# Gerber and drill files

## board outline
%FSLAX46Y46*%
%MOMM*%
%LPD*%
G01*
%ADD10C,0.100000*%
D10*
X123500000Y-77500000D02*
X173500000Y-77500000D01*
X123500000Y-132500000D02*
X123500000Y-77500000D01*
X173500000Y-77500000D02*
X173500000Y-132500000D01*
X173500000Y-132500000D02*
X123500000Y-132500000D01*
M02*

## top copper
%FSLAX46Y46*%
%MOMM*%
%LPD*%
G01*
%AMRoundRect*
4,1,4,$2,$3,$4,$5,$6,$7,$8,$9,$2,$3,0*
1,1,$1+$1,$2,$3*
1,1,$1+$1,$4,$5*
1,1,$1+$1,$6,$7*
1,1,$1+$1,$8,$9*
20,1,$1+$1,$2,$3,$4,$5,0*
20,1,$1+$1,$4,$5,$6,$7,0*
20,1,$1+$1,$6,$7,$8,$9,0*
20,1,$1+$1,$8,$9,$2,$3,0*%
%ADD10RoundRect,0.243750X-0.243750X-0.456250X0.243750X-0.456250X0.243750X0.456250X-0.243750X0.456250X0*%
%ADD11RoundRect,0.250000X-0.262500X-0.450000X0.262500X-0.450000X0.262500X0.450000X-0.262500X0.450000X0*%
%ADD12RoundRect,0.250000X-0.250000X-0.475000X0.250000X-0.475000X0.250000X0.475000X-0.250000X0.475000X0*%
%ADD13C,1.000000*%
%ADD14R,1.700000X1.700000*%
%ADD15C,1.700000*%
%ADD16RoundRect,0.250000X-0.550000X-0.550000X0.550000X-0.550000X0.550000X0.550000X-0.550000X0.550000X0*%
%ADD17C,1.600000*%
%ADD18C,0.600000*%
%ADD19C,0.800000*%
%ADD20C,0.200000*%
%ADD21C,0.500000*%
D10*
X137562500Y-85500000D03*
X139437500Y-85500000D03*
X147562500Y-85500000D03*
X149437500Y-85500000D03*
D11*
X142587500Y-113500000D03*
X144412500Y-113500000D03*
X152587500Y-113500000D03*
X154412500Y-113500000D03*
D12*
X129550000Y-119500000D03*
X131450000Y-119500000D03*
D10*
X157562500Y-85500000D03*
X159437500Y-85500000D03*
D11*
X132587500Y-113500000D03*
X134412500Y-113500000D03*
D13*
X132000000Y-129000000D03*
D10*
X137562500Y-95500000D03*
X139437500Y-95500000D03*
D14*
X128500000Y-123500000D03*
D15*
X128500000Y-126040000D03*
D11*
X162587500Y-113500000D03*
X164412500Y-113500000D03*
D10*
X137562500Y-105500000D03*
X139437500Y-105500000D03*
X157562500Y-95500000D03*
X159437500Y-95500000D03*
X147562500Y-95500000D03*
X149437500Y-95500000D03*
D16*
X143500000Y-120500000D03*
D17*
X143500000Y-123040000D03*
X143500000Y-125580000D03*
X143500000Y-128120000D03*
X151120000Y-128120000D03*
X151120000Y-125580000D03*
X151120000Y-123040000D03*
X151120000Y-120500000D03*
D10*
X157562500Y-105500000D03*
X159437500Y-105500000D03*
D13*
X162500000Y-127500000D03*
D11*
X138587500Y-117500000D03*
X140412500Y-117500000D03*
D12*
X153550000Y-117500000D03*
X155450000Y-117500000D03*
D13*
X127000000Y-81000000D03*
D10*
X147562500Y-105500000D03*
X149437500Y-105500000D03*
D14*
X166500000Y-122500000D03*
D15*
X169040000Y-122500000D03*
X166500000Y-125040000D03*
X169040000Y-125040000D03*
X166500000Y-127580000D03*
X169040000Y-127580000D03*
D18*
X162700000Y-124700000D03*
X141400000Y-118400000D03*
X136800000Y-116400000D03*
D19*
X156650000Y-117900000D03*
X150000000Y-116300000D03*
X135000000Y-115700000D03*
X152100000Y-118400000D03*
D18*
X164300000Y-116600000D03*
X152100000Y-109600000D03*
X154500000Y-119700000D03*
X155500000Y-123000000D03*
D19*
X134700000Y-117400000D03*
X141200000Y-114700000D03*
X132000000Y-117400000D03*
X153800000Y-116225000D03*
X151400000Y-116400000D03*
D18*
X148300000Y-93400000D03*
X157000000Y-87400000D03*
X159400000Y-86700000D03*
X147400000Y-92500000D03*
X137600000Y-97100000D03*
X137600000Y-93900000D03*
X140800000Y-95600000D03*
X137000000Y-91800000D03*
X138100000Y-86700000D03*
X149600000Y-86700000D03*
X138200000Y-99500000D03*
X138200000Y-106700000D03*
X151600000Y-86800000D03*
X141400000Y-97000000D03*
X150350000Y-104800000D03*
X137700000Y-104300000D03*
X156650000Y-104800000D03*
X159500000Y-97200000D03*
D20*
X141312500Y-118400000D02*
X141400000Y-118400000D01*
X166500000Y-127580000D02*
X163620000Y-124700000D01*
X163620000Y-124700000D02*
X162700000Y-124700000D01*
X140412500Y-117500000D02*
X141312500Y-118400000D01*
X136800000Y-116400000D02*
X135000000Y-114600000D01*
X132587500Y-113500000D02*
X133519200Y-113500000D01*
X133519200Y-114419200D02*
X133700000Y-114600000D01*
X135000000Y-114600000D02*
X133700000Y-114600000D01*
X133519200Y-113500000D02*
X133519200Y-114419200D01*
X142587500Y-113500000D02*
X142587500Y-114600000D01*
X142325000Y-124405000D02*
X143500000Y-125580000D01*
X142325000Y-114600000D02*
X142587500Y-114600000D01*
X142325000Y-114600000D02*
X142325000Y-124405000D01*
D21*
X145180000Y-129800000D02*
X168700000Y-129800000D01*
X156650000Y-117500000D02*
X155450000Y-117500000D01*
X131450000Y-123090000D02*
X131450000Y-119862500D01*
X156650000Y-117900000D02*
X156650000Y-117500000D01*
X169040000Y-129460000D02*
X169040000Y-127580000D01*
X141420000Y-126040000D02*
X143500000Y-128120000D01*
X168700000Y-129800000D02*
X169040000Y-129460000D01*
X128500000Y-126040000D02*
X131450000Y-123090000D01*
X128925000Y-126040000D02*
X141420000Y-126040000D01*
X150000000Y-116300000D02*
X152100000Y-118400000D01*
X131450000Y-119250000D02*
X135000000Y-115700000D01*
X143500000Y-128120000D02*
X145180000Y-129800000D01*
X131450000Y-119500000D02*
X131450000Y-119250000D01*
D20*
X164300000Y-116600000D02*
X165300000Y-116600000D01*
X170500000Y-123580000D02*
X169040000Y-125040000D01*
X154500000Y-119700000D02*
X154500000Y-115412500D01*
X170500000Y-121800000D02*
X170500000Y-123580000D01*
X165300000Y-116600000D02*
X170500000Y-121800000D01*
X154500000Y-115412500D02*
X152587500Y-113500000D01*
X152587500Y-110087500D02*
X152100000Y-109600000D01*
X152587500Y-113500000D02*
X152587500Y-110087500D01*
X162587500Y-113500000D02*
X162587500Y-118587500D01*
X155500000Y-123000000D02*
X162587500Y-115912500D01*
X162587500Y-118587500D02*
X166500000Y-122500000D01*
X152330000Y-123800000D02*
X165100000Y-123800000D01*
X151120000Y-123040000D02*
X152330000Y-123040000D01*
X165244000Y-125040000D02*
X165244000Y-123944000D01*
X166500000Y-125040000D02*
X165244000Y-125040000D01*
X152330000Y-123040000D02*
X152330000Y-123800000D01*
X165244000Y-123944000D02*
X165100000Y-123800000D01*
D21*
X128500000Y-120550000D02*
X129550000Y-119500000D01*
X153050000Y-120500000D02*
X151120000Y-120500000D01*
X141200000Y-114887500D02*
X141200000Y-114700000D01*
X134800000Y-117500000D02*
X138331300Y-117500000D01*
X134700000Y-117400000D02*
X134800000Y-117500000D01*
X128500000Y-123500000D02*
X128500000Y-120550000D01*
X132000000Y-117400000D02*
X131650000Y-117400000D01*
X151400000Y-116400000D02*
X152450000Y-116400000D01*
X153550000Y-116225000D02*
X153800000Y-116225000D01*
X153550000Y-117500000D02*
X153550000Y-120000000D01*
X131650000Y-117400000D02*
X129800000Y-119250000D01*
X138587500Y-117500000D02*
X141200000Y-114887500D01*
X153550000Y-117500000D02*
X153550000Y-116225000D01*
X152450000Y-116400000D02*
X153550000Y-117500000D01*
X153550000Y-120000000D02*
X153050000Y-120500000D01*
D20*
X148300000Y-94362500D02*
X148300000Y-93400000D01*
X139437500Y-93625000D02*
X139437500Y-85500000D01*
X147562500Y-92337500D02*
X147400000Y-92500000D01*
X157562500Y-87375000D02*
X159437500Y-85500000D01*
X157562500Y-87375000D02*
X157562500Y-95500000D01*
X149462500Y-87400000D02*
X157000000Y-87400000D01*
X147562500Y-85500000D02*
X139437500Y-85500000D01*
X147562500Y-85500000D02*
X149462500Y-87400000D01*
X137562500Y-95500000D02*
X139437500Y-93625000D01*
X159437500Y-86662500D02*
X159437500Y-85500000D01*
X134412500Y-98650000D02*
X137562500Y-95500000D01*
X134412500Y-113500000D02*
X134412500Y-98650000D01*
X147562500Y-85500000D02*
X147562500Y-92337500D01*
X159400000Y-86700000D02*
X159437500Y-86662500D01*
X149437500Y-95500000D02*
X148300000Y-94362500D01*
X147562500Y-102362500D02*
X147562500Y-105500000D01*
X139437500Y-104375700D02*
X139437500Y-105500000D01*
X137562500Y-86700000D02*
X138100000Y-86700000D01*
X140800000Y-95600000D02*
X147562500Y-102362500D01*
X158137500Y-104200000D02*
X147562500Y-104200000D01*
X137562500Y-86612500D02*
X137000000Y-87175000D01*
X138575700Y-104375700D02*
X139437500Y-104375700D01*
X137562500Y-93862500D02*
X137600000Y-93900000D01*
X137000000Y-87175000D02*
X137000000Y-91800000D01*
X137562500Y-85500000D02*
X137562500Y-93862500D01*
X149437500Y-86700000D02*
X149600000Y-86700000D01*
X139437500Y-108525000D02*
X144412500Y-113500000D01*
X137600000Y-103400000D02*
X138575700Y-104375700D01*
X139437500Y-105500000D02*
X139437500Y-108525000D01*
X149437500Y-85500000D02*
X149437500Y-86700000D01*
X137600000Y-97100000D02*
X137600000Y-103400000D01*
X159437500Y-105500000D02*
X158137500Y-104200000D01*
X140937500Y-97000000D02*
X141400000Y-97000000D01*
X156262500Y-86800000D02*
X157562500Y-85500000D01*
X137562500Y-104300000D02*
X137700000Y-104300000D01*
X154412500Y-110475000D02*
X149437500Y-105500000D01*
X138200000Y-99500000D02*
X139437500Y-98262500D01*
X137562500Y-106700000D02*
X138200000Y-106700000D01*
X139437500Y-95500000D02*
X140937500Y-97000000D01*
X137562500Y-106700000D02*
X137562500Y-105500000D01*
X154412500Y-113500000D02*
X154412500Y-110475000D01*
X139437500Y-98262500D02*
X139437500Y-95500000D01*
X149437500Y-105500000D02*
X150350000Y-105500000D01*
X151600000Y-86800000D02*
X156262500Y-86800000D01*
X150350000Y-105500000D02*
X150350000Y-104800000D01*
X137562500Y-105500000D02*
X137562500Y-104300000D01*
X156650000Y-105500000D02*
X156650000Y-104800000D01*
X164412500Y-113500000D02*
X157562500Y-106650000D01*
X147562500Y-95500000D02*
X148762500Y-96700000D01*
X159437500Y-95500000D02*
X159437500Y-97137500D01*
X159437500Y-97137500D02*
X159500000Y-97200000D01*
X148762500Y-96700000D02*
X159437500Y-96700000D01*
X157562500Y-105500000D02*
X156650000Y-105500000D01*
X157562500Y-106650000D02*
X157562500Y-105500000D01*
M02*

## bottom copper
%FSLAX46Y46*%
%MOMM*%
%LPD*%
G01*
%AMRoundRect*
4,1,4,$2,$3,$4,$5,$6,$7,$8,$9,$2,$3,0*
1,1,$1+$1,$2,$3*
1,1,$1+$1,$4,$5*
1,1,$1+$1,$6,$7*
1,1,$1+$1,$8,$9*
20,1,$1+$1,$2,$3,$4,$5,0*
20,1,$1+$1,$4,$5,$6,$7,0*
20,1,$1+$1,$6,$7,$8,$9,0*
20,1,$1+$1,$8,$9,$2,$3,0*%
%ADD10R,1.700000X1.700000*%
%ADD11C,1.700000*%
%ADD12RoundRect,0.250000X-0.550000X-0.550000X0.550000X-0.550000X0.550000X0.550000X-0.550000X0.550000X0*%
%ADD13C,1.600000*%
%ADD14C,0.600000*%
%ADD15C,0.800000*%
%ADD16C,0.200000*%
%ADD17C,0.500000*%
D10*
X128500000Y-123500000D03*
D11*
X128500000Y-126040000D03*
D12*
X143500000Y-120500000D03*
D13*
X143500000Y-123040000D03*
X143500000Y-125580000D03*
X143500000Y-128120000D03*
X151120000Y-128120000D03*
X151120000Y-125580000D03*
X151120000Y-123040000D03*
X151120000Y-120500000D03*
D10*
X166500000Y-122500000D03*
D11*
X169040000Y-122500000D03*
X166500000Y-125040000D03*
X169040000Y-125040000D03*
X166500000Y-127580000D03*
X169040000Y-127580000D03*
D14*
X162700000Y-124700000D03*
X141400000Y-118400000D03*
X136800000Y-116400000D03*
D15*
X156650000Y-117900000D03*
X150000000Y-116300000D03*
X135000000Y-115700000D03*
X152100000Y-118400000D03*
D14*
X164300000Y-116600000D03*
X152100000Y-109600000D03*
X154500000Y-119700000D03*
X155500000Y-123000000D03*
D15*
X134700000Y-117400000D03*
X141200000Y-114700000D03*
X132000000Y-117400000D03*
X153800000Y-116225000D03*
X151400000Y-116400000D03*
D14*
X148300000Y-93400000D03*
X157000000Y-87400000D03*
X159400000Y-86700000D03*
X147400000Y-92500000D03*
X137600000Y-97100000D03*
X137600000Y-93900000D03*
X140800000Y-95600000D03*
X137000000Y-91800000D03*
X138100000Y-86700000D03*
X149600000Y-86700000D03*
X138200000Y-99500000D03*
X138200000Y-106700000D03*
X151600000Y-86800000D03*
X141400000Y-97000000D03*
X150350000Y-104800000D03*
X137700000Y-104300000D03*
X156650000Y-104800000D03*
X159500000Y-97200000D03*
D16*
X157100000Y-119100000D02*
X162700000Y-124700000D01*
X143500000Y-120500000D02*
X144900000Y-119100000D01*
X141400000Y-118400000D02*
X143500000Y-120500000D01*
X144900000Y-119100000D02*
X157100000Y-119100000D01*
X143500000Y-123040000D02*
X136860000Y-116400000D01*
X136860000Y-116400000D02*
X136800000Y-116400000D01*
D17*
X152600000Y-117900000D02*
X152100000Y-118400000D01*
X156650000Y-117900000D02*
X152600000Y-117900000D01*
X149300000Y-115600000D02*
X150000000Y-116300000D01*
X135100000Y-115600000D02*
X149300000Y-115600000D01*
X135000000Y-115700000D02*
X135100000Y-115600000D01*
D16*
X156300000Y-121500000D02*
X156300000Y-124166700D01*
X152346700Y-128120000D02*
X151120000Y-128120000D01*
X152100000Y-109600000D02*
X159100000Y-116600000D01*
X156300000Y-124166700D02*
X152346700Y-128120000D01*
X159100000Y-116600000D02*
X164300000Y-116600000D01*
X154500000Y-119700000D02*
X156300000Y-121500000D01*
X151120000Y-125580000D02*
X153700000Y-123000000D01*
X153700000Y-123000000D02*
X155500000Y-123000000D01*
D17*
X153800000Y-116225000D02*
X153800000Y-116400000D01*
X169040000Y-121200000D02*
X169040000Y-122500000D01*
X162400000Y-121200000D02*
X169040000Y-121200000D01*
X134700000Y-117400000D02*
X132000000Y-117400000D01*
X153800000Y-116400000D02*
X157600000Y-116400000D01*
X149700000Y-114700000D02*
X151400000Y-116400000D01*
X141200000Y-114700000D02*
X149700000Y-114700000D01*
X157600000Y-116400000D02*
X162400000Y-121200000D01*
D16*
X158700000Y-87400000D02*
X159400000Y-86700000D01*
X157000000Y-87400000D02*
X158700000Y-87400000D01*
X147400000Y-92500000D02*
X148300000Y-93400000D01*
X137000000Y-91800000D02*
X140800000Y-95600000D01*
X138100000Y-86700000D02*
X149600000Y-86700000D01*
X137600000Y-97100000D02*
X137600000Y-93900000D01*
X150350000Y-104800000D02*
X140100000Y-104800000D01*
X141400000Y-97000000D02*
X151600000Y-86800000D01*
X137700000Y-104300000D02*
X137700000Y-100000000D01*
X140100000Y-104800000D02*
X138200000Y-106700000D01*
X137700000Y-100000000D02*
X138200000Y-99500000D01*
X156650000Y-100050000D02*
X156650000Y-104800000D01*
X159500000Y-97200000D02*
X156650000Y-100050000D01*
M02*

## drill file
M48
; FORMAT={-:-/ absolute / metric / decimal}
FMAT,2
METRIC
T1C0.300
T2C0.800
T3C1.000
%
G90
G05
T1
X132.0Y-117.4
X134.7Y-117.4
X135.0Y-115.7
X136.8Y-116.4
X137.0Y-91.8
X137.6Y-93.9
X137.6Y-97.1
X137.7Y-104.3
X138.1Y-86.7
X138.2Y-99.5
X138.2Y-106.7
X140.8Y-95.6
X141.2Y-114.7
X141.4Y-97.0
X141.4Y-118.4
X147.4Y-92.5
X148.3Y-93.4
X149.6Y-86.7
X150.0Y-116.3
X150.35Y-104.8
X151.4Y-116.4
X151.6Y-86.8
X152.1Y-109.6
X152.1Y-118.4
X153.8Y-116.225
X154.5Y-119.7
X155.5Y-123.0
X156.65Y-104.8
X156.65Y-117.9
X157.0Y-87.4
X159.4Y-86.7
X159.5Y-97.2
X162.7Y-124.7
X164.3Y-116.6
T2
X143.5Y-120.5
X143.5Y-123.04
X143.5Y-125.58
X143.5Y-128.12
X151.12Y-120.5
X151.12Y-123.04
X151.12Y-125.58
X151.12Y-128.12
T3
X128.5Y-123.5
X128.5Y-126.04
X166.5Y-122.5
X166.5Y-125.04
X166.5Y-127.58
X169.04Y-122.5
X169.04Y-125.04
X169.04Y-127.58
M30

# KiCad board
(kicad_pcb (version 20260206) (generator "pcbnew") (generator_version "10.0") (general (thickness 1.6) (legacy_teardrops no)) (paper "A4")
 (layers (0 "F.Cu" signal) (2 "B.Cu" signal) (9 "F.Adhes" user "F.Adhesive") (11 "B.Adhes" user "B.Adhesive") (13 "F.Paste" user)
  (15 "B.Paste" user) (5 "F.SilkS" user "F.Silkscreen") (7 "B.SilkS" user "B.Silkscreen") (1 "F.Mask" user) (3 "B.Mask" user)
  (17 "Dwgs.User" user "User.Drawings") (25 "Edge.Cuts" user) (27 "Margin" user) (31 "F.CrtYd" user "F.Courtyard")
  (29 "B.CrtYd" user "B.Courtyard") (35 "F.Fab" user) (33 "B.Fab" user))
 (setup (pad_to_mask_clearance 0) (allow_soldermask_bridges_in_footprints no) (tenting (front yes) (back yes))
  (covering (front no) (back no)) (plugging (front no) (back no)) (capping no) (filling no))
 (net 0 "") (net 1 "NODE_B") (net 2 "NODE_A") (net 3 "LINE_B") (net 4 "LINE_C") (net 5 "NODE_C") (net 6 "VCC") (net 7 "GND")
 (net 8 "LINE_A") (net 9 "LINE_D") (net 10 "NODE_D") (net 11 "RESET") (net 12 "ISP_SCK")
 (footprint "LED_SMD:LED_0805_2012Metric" (layer "F.Cu") (at 138.5 85.5)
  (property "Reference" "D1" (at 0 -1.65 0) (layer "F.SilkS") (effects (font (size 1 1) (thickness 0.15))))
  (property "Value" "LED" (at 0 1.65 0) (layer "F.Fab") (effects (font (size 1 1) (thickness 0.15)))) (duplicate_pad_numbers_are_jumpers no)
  (pad "1" smd roundrect (at -0.9375 0) (size 0.975 1.4) (layers "F.Cu" "F.Mask" "F.Paste") (roundrect_rratio 0.25) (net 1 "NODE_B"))
  (pad "2" smd roundrect (at 0.9375 0) (size 0.975 1.4) (layers "F.Cu" "F.Mask" "F.Paste") (roundrect_rratio 0.25) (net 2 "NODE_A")))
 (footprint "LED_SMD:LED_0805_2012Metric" (layer "F.Cu") (at 148.5 85.5)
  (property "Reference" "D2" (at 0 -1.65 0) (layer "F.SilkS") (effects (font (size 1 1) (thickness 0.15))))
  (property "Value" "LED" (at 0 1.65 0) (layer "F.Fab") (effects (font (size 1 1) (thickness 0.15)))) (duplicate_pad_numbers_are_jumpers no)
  (pad "1" smd roundrect (at -0.9375 0) (size 0.975 1.4) (layers "F.Cu" "F.Mask" "F.Paste") (roundrect_rratio 0.25) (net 2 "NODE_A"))
  (pad "2" smd roundrect (at 0.9375 0) (size 0.975 1.4) (layers "F.Cu" "F.Mask" "F.Paste") (roundrect_rratio 0.25) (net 1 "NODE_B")))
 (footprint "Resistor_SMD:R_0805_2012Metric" (layer "F.Cu") (at 143.5 113.5)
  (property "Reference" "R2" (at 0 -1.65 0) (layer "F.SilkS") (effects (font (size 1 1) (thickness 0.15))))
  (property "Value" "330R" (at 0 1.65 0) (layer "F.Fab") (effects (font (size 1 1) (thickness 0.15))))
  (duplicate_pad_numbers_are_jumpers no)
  (pad "1" smd roundrect (at -0.9125 0) (size 1.025 1.4) (layers "F.Cu" "F.Mask" "F.Paste") (roundrect_rratio 0.243902) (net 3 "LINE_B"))
  (pad "2" smd roundrect (at 0.9125 0) (size 1.025 1.4) (layers "F.Cu" "F.Mask" "F.Paste") (roundrect_rratio 0.243902) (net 1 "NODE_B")))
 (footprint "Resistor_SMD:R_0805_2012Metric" (layer "F.Cu") (at 153.5 113.5)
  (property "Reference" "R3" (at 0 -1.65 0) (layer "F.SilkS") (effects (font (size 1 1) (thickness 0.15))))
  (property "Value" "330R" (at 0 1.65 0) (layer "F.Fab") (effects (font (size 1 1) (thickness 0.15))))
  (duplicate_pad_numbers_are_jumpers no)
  (pad "1" smd roundrect (at -0.9125 0) (size 1.025 1.4) (layers "F.Cu" "F.Mask" "F.Paste") (roundrect_rratio 0.243902) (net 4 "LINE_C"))
  (pad "2" smd roundrect (at 0.9125 0) (size 1.025 1.4) (layers "F.Cu" "F.Mask" "F.Paste") (roundrect_rratio 0.243902) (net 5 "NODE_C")))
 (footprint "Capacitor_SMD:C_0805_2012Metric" (layer "F.Cu") (at 130.5 119.5)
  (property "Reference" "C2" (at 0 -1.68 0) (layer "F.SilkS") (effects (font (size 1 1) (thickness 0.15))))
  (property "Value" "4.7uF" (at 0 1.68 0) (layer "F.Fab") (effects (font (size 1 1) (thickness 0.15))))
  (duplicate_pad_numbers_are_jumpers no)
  (pad "1" smd roundrect (at -0.95 0) (size 1 1.45) (layers "F.Cu" "F.Mask" "F.Paste") (roundrect_rratio 0.25) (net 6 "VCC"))
  (pad "2" smd roundrect (at 0.95 0) (size 1 1.45) (layers "F.Cu" "F.Mask" "F.Paste") (roundrect_rratio 0.25) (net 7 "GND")))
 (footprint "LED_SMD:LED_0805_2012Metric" (layer "F.Cu") (at 158.5 85.5)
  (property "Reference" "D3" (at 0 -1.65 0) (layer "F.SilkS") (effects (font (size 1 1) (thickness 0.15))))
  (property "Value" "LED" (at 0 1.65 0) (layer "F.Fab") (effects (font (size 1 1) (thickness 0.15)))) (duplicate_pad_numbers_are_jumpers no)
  (pad "1" smd roundrect (at -0.9375 0) (size 0.975 1.4) (layers "F.Cu" "F.Mask" "F.Paste") (roundrect_rratio 0.25) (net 5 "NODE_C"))
  (pad "2" smd roundrect (at 0.9375 0) (size 0.975 1.4) (layers "F.Cu" "F.Mask" "F.Paste") (roundrect_rratio 0.25) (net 2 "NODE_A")))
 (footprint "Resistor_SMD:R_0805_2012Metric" (layer "F.Cu") (at 133.5 113.5)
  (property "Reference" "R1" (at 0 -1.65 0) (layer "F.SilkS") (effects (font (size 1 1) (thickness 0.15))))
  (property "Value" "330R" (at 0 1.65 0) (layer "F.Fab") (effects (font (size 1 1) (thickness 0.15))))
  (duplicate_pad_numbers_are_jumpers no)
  (pad "1" smd roundrect (at -0.9125 0) (size 1.025 1.4) (layers "F.Cu" "F.Mask" "F.Paste") (roundrect_rratio 0.243902) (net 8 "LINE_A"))
  (pad "2" smd roundrect (at 0.9125 0) (size 1.025 1.4) (layers "F.Cu" "F.Mask" "F.Paste") (roundrect_rratio 0.243902) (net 2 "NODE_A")))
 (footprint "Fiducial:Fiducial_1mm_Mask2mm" (layer "F.Cu") (at 132 129)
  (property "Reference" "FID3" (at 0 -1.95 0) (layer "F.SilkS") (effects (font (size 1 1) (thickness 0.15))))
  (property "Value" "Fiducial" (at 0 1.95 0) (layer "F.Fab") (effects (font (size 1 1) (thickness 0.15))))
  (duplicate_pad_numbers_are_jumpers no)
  (pad "" smd circle (at 0 0) (size 1 1) (layers "F.Cu" "F.Mask") (solder_mask_margin 0.5) (clearance 0.6)))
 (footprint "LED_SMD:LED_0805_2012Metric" (layer "F.Cu") (at 138.5 95.5)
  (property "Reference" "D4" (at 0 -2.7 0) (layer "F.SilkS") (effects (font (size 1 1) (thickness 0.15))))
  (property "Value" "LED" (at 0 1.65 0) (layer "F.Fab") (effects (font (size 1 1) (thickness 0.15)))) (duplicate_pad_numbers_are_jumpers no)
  (pad "1" smd roundrect (at -0.9375 0) (size 0.975 1.4) (layers "F.Cu" "F.Mask" "F.Paste") (roundrect_rratio 0.25) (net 2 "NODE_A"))
  (pad "2" smd roundrect (at 0.9375 0) (size 0.975 1.4) (layers "F.Cu" "F.Mask" "F.Paste") (roundrect_rratio 0.25) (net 5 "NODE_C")))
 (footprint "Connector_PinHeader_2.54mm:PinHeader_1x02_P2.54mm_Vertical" (layer "F.Cu") (at 128.5 123.5)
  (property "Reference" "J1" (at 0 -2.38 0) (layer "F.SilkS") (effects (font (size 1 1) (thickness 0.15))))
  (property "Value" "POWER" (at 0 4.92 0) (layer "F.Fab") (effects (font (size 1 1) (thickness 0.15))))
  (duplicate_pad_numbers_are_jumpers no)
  (pad "1" thru_hole rect (at 0 0) (size 1.7 1.7) (drill 1) (layers "*.Cu" "*.Mask") (remove_unused_layers no) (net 6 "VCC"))
  (pad "2" thru_hole circle (at 0 2.54) (size 1.7 1.7) (drill 1) (layers "*.Cu" "*.Mask") (remove_unused_layers no) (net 7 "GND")))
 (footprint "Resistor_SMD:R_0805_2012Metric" (layer "F.Cu") (at 163.5 113.5)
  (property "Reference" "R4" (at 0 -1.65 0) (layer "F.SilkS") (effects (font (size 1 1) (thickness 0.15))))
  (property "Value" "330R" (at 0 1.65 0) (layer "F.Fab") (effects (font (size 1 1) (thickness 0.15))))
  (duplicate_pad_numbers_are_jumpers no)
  (pad "1" smd roundrect (at -0.9125 0) (size 1.025 1.4) (layers "F.Cu" "F.Mask" "F.Paste") (roundrect_rratio 0.243902) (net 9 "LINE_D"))
  (pad "2" smd roundrect (at 0.9125 0) (size 1.025 1.4) (layers "F.Cu" "F.Mask" "F.Paste") (roundrect_rratio 0.243902) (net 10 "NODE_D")))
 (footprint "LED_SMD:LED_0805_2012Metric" (layer "F.Cu") (at 138.5 105.5)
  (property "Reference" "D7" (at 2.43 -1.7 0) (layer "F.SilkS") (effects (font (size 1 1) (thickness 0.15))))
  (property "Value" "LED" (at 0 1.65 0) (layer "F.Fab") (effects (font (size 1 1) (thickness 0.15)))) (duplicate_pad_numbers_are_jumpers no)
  (pad "1" smd roundrect (at -0.9375 0) (size 0.975 1.4) (layers "F.Cu" "F.Mask" "F.Paste") (roundrect_rratio 0.25) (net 5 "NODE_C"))
  (pad "2" smd roundrect (at 0.9375 0) (size 0.975 1.4) (layers "F.Cu" "F.Mask" "F.Paste") (roundrect_rratio 0.25) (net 1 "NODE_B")))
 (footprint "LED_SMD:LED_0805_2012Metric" (layer "F.Cu") (at 158.5 95.5)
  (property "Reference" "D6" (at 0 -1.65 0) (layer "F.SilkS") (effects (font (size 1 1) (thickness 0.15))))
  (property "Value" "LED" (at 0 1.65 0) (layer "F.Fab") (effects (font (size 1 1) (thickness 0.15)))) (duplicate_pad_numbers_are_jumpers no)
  (pad "1" smd roundrect (at -0.9375 0) (size 0.975 1.4) (layers "F.Cu" "F.Mask" "F.Paste") (roundrect_rratio 0.25) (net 2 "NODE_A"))
  (pad "2" smd roundrect (at 0.9375 0) (size 0.975 1.4) (layers "F.Cu" "F.Mask" "F.Paste") (roundrect_rratio 0.25) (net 10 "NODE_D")))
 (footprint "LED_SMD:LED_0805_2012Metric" (layer "F.Cu") (at 148.5 95.5)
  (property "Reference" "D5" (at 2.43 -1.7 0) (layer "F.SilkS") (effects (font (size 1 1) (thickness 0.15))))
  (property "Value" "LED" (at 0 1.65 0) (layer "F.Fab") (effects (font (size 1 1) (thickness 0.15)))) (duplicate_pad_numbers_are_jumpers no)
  (pad "1" smd roundrect (at -0.9375 0) (size 0.975 1.4) (layers "F.Cu" "F.Mask" "F.Paste") (roundrect_rratio 0.25) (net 10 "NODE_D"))
  (pad "2" smd roundrect (at 0.9375 0) (size 0.975 1.4) (layers "F.Cu" "F.Mask" "F.Paste") (roundrect_rratio 0.25) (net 2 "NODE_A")))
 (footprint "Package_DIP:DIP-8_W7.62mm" (layer "F.Cu") (at 143.5 120.5)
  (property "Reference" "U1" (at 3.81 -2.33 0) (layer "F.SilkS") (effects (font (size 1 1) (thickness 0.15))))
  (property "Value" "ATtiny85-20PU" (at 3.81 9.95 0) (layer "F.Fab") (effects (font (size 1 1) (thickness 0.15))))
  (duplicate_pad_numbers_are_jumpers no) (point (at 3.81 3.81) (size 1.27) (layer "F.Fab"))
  (pad "1" thru_hole roundrect (at 0 0) (size 1.6 1.6) (drill 0.8) (layers "*.Cu" "*.Mask") (remove_unused_layers no)
   (roundrect_rratio 0.15625) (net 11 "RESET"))
  (pad "2" thru_hole circle (at 0 2.54) (size 1.6 1.6) (drill 0.8) (layers "*.Cu" "*.Mask") (remove_unused_layers no) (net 8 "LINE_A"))
  (pad "3" thru_hole circle (at 0 5.08) (size 1.6 1.6) (drill 0.8) (layers "*.Cu" "*.Mask") (remove_unused_layers no) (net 3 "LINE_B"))
  (pad "4" thru_hole circle (at 0 7.62) (size 1.6 1.6) (drill 0.8) (layers "*.Cu" "*.Mask") (remove_unused_layers no) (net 7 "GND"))
  (pad "5" thru_hole circle (at 7.62 7.62) (size 1.6 1.6) (drill 0.8) (layers "*.Cu" "*.Mask") (remove_unused_layers no) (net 4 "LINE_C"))
  (pad "6" thru_hole circle (at 7.62 5.08) (size 1.6 1.6) (drill 0.8) (layers "*.Cu" "*.Mask") (remove_unused_layers no) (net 9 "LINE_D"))
  (pad "7" thru_hole circle (at 7.62 2.54) (size 1.6 1.6) (drill 0.8) (layers "*.Cu" "*.Mask") (remove_unused_layers no) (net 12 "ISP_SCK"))
  (pad "8" thru_hole circle (at 7.62 0) (size 1.6 1.6) (drill 0.8) (layers "*.Cu" "*.Mask") (remove_unused_layers no) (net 6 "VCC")))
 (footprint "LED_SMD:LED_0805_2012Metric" (layer "F.Cu") (at 158.5 105.5)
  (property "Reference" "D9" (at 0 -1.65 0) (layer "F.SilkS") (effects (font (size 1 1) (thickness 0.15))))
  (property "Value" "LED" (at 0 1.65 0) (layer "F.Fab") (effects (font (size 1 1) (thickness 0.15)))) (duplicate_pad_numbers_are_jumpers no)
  (pad "1" smd roundrect (at -0.9375 0) (size 0.975 1.4) (layers "F.Cu" "F.Mask" "F.Paste") (roundrect_rratio 0.25) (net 10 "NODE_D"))
  (pad "2" smd roundrect (at 0.9375 0) (size 0.975 1.4) (layers "F.Cu" "F.Mask" "F.Paste") (roundrect_rratio 0.25) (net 1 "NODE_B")))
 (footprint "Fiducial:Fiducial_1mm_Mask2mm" (layer "F.Cu") (at 162.5 127.5)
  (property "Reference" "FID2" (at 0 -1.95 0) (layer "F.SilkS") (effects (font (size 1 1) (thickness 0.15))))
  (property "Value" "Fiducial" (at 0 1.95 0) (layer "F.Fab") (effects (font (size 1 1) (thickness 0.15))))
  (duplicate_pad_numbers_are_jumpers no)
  (pad "" smd circle (at 0 0) (size 1 1) (layers "F.Cu" "F.Mask") (solder_mask_margin 0.5) (clearance 0.6)))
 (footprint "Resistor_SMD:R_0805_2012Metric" (layer "F.Cu") (at 139.5 117.5)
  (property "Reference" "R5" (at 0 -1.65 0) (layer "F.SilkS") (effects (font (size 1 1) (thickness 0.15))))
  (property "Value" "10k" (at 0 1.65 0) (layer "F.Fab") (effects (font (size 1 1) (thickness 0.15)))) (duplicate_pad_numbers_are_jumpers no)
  (pad "1" smd roundrect (at -0.9125 0) (size 1.025 1.4) (layers "F.Cu" "F.Mask" "F.Paste") (roundrect_rratio 0.243902) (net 6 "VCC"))
  (pad "2" smd roundrect (at 0.9125 0) (size 1.025 1.4) (layers "F.Cu" "F.Mask" "F.Paste") (roundrect_rratio 0.243902) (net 11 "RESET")))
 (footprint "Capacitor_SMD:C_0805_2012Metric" (layer "F.Cu") (at 154.5 117.5)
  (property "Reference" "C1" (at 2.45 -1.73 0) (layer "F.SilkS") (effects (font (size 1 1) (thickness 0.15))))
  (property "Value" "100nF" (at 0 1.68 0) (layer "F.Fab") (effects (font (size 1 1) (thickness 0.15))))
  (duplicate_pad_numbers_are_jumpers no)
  (pad "1" smd roundrect (at -0.95 0) (size 1 1.45) (layers "F.Cu" "F.Mask" "F.Paste") (roundrect_rratio 0.25) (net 6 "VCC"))
  (pad "2" smd roundrect (at 0.95 0) (size 1 1.45) (layers "F.Cu" "F.Mask" "F.Paste") (roundrect_rratio 0.25) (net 7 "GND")))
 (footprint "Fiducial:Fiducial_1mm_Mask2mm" (layer "F.Cu") (at 127 81)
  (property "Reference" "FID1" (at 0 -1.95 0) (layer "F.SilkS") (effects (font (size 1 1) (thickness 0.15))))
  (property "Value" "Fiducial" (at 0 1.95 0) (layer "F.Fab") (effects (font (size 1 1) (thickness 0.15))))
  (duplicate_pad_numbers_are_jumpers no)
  (pad "" smd circle (at 0 0) (size 1 1) (layers "F.Cu" "F.Mask") (solder_mask_margin 0.5) (clearance 0.6)))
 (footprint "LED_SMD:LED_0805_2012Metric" (layer "F.Cu") (at 148.5 105.5)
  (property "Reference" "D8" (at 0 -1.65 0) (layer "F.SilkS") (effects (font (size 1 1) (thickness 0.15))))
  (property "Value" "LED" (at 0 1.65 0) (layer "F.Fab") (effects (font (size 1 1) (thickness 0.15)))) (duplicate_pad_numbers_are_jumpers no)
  (pad "1" smd roundrect (at -0.9375 0) (size 0.975 1.4) (layers "F.Cu" "F.Mask" "F.Paste") (roundrect_rratio 0.25) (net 1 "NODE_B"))
  (pad "2" smd roundrect (at 0.9375 0) (size 0.975 1.4) (layers "F.Cu" "F.Mask" "F.Paste") (roundrect_rratio 0.25) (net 5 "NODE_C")))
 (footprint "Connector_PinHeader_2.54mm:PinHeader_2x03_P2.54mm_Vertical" (layer "F.Cu") (at 166.5 122.5)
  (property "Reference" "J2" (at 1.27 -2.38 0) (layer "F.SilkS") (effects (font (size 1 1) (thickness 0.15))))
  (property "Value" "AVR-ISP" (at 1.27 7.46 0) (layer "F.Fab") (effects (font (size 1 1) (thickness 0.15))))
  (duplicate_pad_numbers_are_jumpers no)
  (pad "1" thru_hole rect (at 0 0) (size 1.7 1.7) (drill 1) (layers "*.Cu" "*.Mask") (remove_unused_layers no) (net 9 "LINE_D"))
  (pad "2" thru_hole circle (at 2.54 0) (size 1.7 1.7) (drill 1) (layers "*.Cu" "*.Mask") (remove_unused_layers no) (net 6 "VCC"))
  (pad "3" thru_hole circle (at 0 2.54) (size 1.7 1.7) (drill 1) (layers "*.Cu" "*.Mask") (remove_unused_layers no) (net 12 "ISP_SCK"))
  (pad "4" thru_hole circle (at 2.54 2.54) (size 1.7 1.7) (drill 1) (layers "*.Cu" "*.Mask") (remove_unused_layers no) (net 4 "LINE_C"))
  (pad "5" thru_hole circle (at 0 5.08) (size 1.7 1.7) (drill 1) (layers "*.Cu" "*.Mask") (remove_unused_layers no) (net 11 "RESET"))
  (pad "6" thru_hole circle (at 2.54 5.08) (size 1.7 1.7) (drill 1) (layers "*.Cu" "*.Mask") (remove_unused_layers no) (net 7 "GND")))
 (gr_line (start 123.5 77.5) (end 173.5 77.5) (stroke (width 0.1) (type default)) (layer "Edge.Cuts"))
 (gr_line (start 123.5 132.5) (end 123.5 77.5) (stroke (width 0.1) (type default)) (layer "Edge.Cuts"))
 (gr_line (start 173.5 77.5) (end 173.5 132.5) (stroke (width 0.1) (type default)) (layer "Edge.Cuts"))
 (gr_line (start 173.5 132.5) (end 123.5 132.5) (stroke (width 0.1) (type default)) (layer "Edge.Cuts"))
 (segment (start 141.3125 118.4) (end 141.4 118.4) (width 0.2) (layer "F.Cu") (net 11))
 (segment (start 166.5 127.58) (end 163.62 124.7) (width 0.2) (layer "F.Cu") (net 11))
 (segment (start 163.62 124.7) (end 162.7 124.7) (width 0.2) (layer "F.Cu") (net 11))
 (segment (start 140.4125 117.5) (end 141.3125 118.4) (width 0.2) (layer "F.Cu") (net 11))
 (via (at 162.7 124.7) (size 0.6) (drill 0.3) (layers "F.Cu" "B.Cu") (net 11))
 (via (at 141.4 118.4) (size 0.6) (drill 0.3) (layers "F.Cu" "B.Cu") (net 11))
 (segment (start 157.1 119.1) (end 162.7 124.7) (width 0.2) (layer "B.Cu") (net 11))
 (segment (start 143.5 120.5) (end 144.9 119.1) (width 0.2) (layer "B.Cu") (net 11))
 (segment (start 141.4 118.4) (end 143.5 120.5) (width 0.2) (layer "B.Cu") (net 11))
 (segment (start 144.9 119.1) (end 157.1 119.1) (width 0.2) (layer "B.Cu") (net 11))
 (segment (start 136.8 116.4) (end 135 114.6) (width 0.2) (layer "F.Cu") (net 8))
 (segment (start 132.5875 113.5) (end 133.5192 113.5) (width 0.2) (layer "F.Cu") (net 8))
 (segment (start 133.5192 114.4192) (end 133.7 114.6) (width 0.2) (layer "F.Cu") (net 8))
 (segment (start 135 114.6) (end 133.7 114.6) (width 0.2) (layer "F.Cu") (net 8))
 (segment (start 133.5192 113.5) (end 133.5192 114.4192) (width 0.2) (layer "F.Cu") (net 8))
 (via (at 136.8 116.4) (size 0.6) (drill 0.3) (layers "F.Cu" "B.Cu") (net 8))
 (segment (start 143.5 123.04) (end 136.86 116.4) (width 0.2) (layer "B.Cu") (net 8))
 (segment (start 136.86 116.4) (end 136.8 116.4) (width 0.2) (layer "B.Cu") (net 8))
 (segment (start 142.5875 113.5) (end 142.5875 114.6) (width 0.2) (layer "F.Cu") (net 3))
 (segment (start 142.325 124.405) (end 143.5 125.58) (width 0.2) (layer "F.Cu") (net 3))
 (segment (start 142.325 114.6) (end 142.5875 114.6) (width 0.2) (layer "F.Cu") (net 3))
 (segment (start 142.325 114.6) (end 142.325 124.405) (width 0.2) (layer "F.Cu") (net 3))
 (segment (start 145.18 129.8) (end 168.7 129.8) (width 0.5) (layer "F.Cu") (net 7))
 (segment (start 156.65 117.5) (end 155.45 117.5) (width 0.5) (layer "F.Cu") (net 7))
 (segment (start 131.45 123.09) (end 131.45 119.8625) (width 0.5) (layer "F.Cu") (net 7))
 (segment (start 156.65 117.9) (end 156.65 117.5) (width 0.5) (layer "F.Cu") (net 7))
 (segment (start 169.04 129.46) (end 169.04 127.58) (width 0.5) (layer "F.Cu") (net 7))
 (segment (start 141.42 126.04) (end 143.5 128.12) (width 0.5) (layer "F.Cu") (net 7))
 (segment (start 168.7 129.8) (end 169.04 129.46) (width 0.5) (layer "F.Cu") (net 7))
 (segment (start 128.5 126.04) (end 131.45 123.09) (width 0.5) (layer "F.Cu") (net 7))
 (segment (start 128.925 126.04) (end 141.42 126.04) (width 0.5) (layer "F.Cu") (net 7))
 (segment (start 150 116.3) (end 152.1 118.4) (width 0.5) (layer "F.Cu") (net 7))
 (segment (start 131.45 119.25) (end 135 115.7) (width 0.5) (layer "F.Cu") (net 7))
 (segment (start 143.5 128.12) (end 145.18 129.8) (width 0.5) (layer "F.Cu") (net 7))
 (segment (start 131.45 119.5) (end 131.45 119.25) (width 0.5) (layer "F.Cu") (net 7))
 (via (at 156.65 117.9) (size 0.8) (drill 0.3) (layers "F.Cu" "B.Cu") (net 7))
 (via (at 150 116.3) (size 0.8) (drill 0.3) (layers "F.Cu" "B.Cu") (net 7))
 (via (at 135 115.7) (size 0.8) (drill 0.3) (layers "F.Cu" "B.Cu") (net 7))
 (via (at 152.1 118.4) (size 0.8) (drill 0.3) (layers "F.Cu" "B.Cu") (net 7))
 (segment (start 152.6 117.9) (end 152.1 118.4) (width 0.5) (layer "B.Cu") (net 7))
 (segment (start 156.65 117.9) (end 152.6 117.9) (width 0.5) (layer "B.Cu") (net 7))
 (segment (start 149.3 115.6) (end 150 116.3) (width 0.5) (layer "B.Cu") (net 7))
 (segment (start 135.1 115.6) (end 149.3 115.6) (width 0.5) (layer "B.Cu") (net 7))
 (segment (start 135 115.7) (end 135.1 115.6) (width 0.5) (layer "B.Cu") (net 7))
 (segment (start 164.3 116.6) (end 165.3 116.6) (width 0.2) (layer "F.Cu") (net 4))
 (segment (start 170.5 123.58) (end 169.04 125.04) (width 0.2) (layer "F.Cu") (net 4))
 (segment (start 154.5 119.7) (end 154.5 115.4125) (width 0.2) (layer "F.Cu") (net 4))
 (segment (start 170.5 121.8) (end 170.5 123.58) (width 0.2) (layer "F.Cu") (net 4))
 (segment (start 165.3 116.6) (end 170.5 121.8) (width 0.2) (layer "F.Cu") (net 4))
 (segment (start 154.5 115.4125) (end 152.5875 113.5) (width 0.2) (layer "F.Cu") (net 4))
 (segment (start 152.5875 110.0875) (end 152.1 109.6) (width 0.2) (layer "F.Cu") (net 4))
 (segment (start 152.5875 113.5) (end 152.5875 110.0875) (width 0.2) (layer "F.Cu") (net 4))
 (via (at 164.3 116.6) (size 0.6) (drill 0.3) (layers "F.Cu" "B.Cu") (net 4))
 (via (at 152.1 109.6) (size 0.6) (drill 0.3) (layers "F.Cu" "B.Cu") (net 4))
 (via (at 154.5 119.7) (size 0.6) (drill 0.3) (layers "F.Cu" "B.Cu") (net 4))
 (segment (start 156.3 121.5) (end 156.3 124.1667) (width 0.2) (layer "B.Cu") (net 4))
 (segment (start 152.3467 128.12) (end 151.12 128.12) (width 0.2) (layer "B.Cu") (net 4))
 (segment (start 152.1 109.6) (end 159.1 116.6) (width 0.2) (layer "B.Cu") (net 4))
 (segment (start 156.3 124.1667) (end 152.3467 128.12) (width 0.2) (layer "B.Cu") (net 4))
 (segment (start 159.1 116.6) (end 164.3 116.6) (width 0.2) (layer "B.Cu") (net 4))
 (segment (start 154.5 119.7) (end 156.3 121.5) (width 0.2) (layer "B.Cu") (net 4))
 (segment (start 162.5875 113.5) (end 162.5875 118.5875) (width 0.2) (layer "F.Cu") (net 9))
 (segment (start 155.5 123) (end 162.5875 115.9125) (width 0.2) (layer "F.Cu") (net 9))
 (segment (start 162.5875 118.5875) (end 166.5 122.5) (width 0.2) (layer "F.Cu") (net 9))
 (via (at 155.5 123) (size 0.6) (drill 0.3) (layers "F.Cu" "B.Cu") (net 9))
 (segment (start 151.12 125.58) (end 153.7 123) (width 0.2) (layer "B.Cu") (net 9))
 (segment (start 153.7 123) (end 155.5 123) (width 0.2) (layer "B.Cu") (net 9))
 (segment (start 152.33 123.8) (end 165.1 123.8) (width 0.2) (layer "F.Cu") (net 12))
 (segment (start 151.12 123.04) (end 152.33 123.04) (width 0.2) (layer "F.Cu") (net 12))
 (segment (start 165.244 125.04) (end 165.244 123.944) (width 0.2) (layer "F.Cu") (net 12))
 (segment (start 166.5 125.04) (end 165.244 125.04) (width 0.2) (layer "F.Cu") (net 12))
 (segment (start 152.33 123.04) (end 152.33 123.8) (width 0.2) (layer "F.Cu") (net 12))
 (segment (start 165.244 123.944) (end 165.1 123.8) (width 0.2) (layer "F.Cu") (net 12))
 (segment (start 128.5 120.55) (end 129.55 119.5) (width 0.5) (layer "F.Cu") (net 6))
 (segment (start 153.05 120.5) (end 151.12 120.5) (width 0.5) (layer "F.Cu") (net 6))
 (segment (start 141.2 114.8875) (end 141.2 114.7) (width 0.5) (layer "F.Cu") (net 6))
 (segment (start 134.8 117.5) (end 138.3313 117.5) (width 0.5) (layer "F.Cu") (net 6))
 (segment (start 134.7 117.4) (end 134.8 117.5) (width 0.5) (layer "F.Cu") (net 6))
 (segment (start 128.5 123.5) (end 128.5 120.55) (width 0.5) (layer "F.Cu") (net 6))
 (segment (start 132 117.4) (end 131.65 117.4) (width 0.5) (layer "F.Cu") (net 6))
 (segment (start 151.4 116.4) (end 152.45 116.4) (width 0.5) (layer "F.Cu") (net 6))
 (segment (start 153.55 116.225) (end 153.8 116.225) (width 0.5) (layer "F.Cu") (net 6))
 (segment (start 153.55 117.5) (end 153.55 120) (width 0.5) (layer "F.Cu") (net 6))
 (segment (start 131.65 117.4) (end 129.8 119.25) (width 0.5) (layer "F.Cu") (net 6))
 (segment (start 138.5875 117.5) (end 141.2 114.8875) (width 0.5) (layer "F.Cu") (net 6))
 (segment (start 153.55 117.5) (end 153.55 116.225) (width 0.5) (layer "F.Cu") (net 6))
 (segment (start 152.45 116.4) (end 153.55 117.5) (width 0.5) (layer "F.Cu") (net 6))
 (segment (start 153.55 120) (end 153.05 120.5) (width 0.5) (layer "F.Cu") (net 6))
 (via (at 134.7 117.4) (size 0.8) (drill 0.3) (layers "F.Cu" "B.Cu") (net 6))
 (via (at 141.2 114.7) (size 0.8) (drill 0.3) (layers "F.Cu" "B.Cu") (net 6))
 (via (at 132 117.4) (size 0.8) (drill 0.3) (layers "F.Cu" "B.Cu") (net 6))
 (via (at 153.8 116.225) (size 0.8) (drill 0.3) (layers "F.Cu" "B.Cu") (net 6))
 (via (at 151.4 116.4) (size 0.8) (drill 0.3) (layers "F.Cu" "B.Cu") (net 6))
 (segment (start 153.8 116.225) (end 153.8 116.4) (width 0.5) (layer "B.Cu") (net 6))
 (segment (start 169.04 121.2) (end 169.04 122.5) (width 0.5) (layer "B.Cu") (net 6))
 (segment (start 162.4 121.2) (end 169.04 121.2) (width 0.5) (layer "B.Cu") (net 6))
 (segment (start 134.7 117.4) (end 132 117.4) (width 0.5) (layer "B.Cu") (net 6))
 (segment (start 153.8 116.4) (end 157.6 116.4) (width 0.5) (layer "B.Cu") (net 6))
 (segment (start 149.7 114.7) (end 151.4 116.4) (width 0.5) (layer "B.Cu") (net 6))
 (segment (start 141.2 114.7) (end 149.7 114.7) (width 0.5) (layer "B.Cu") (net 6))
 (segment (start 157.6 116.4) (end 162.4 121.2) (width 0.5) (layer "B.Cu") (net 6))
 (segment (start 148.3 94.3625) (end 148.3 93.4) (width 0.2) (layer "F.Cu") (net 2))
 (segment (start 139.4375 93.625) (end 139.4375 85.5) (width 0.2) (layer "F.Cu") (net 2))
 (segment (start 147.5625 92.3375) (end 147.4 92.5) (width 0.2) (layer "F.Cu") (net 2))
 (segment (start 157.5625 87.375) (end 159.4375 85.5) (width 0.2) (layer "F.Cu") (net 2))
 (segment (start 157.5625 87.375) (end 157.5625 95.5) (width 0.2) (layer "F.Cu") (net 2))
 (segment (start 149.4625 87.4) (end 157 87.4) (width 0.2) (layer "F.Cu") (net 2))
 (segment (start 147.5625 85.5) (end 139.4375 85.5) (width 0.2) (layer "F.Cu") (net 2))
 (segment (start 147.5625 85.5) (end 149.4625 87.4) (width 0.2) (layer "F.Cu") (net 2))
 (segment (start 137.5625 95.5) (end 139.4375 93.625) (width 0.2) (layer "F.Cu") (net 2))
 (segment (start 159.4375 86.6625) (end 159.4375 85.5) (width 0.2) (layer "F.Cu") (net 2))
 (segment (start 134.4125 98.65) (end 137.5625 95.5) (width 0.2) (layer "F.Cu") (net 2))
 (segment (start 134.4125 113.5) (end 134.4125 98.65) (width 0.2) (layer "F.Cu") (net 2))
 (segment (start 147.5625 85.5) (end 147.5625 92.3375) (width 0.2) (layer "F.Cu") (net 2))
 (segment (start 159.4 86.7) (end 159.4375 86.6625) (width 0.2) (layer "F.Cu") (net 2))
 (segment (start 149.4375 95.5) (end 148.3 94.3625) (width 0.2) (layer "F.Cu") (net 2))
 (via (at 148.3 93.4) (size 0.6) (drill 0.3) (layers "F.Cu" "B.Cu") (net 2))
 (via (at 157 87.4) (size 0.6) (drill 0.3) (layers "F.Cu" "B.Cu") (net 2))
 (via (at 159.4 86.7) (size 0.6) (drill 0.3) (layers "F.Cu" "B.Cu") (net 2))
 (via (at 147.4 92.5) (size 0.6) (drill 0.3) (layers "F.Cu" "B.Cu") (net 2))
 (segment (start 158.7 87.4) (end 159.4 86.7) (width 0.2) (layer "B.Cu") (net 2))
 (segment (start 157 87.4) (end 158.7 87.4) (width 0.2) (layer "B.Cu") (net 2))
 (segment (start 147.4 92.5) (end 148.3 93.4) (width 0.2) (layer "B.Cu") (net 2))
 (segment (start 147.5625 102.3625) (end 147.5625 105.5) (width 0.2) (layer "F.Cu") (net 1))
 (segment (start 139.4375 104.3757) (end 139.4375 105.5) (width 0.2) (layer "F.Cu") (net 1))
 (segment (start 137.5625 86.7) (end 138.1 86.7) (width 0.2) (layer "F.Cu") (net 1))
 (segment (start 140.8 95.6) (end 147.5625 102.3625) (width 0.2) (layer "F.Cu") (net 1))
 (segment (start 158.1375 104.2) (end 147.5625 104.2) (width 0.2) (layer "F.Cu") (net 1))
 (segment (start 137.5625 86.6125) (end 137 87.175) (width 0.2) (layer "F.Cu") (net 1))
 (segment (start 138.5757 104.3757) (end 139.4375 104.3757) (width 0.2) (layer "F.Cu") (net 1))
 (segment (start 137.5625 93.8625) (end 137.6 93.9) (width 0.2) (layer "F.Cu") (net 1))
 (segment (start 137 87.175) (end 137 91.8) (width 0.2) (layer "F.Cu") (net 1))
 (segment (start 137.5625 85.5) (end 137.5625 93.8625) (width 0.2) (layer "F.Cu") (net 1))
 (segment (start 149.4375 86.7) (end 149.6 86.7) (width 0.2) (layer "F.Cu") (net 1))
 (segment (start 139.4375 108.525) (end 144.4125 113.5) (width 0.2) (layer "F.Cu") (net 1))
 (segment (start 137.6 103.4) (end 138.5757 104.3757) (width 0.2) (layer "F.Cu") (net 1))
 (segment (start 139.4375 105.5) (end 139.4375 108.525) (width 0.2) (layer "F.Cu") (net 1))
 (segment (start 149.4375 85.5) (end 149.4375 86.7) (width 0.2) (layer "F.Cu") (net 1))
 (segment (start 137.6 97.1) (end 137.6 103.4) (width 0.2) (layer "F.Cu") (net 1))
 (segment (start 159.4375 105.5) (end 158.1375 104.2) (width 0.2) (layer "F.Cu") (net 1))
 (via (at 137.6 97.1) (size 0.6) (drill 0.3) (layers "F.Cu" "B.Cu") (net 1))
 (via (at 137.6 93.9) (size 0.6) (drill 0.3) (layers "F.Cu" "B.Cu") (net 1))
 (via (at 140.8 95.6) (size 0.6) (drill 0.3) (layers "F.Cu" "B.Cu") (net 1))
 (via (at 137 91.8) (size 0.6) (drill 0.3) (layers "F.Cu" "B.Cu") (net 1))
 (via (at 138.1 86.7) (size 0.6) (drill 0.3) (layers "F.Cu" "B.Cu") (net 1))
 (via (at 149.6 86.7) (size 0.6) (drill 0.3) (layers "F.Cu" "B.Cu") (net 1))
 (segment (start 137 91.8) (end 140.8 95.6) (width 0.2) (layer "B.Cu") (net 1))
 (segment (start 138.1 86.7) (end 149.6 86.7) (width 0.2) (layer "B.Cu") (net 1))
 (segment (start 137.6 97.1) (end 137.6 93.9) (width 0.2) (layer "B.Cu") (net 1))
 (segment (start 140.9375 97) (end 141.4 97) (width 0.2) (layer "F.Cu") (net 5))
 (segment (start 156.2625 86.8) (end 157.5625 85.5) (width 0.2) (layer "F.Cu") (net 5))
 (segment (start 137.5625 104.3) (end 137.7 104.3) (width 0.2) (layer "F.Cu") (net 5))
 (segment (start 154.4125 110.475) (end 149.4375 105.5) (width 0.2) (layer "F.Cu") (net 5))
 (segment (start 138.2 99.5) (end 139.4375 98.2625) (width 0.2) (layer "F.Cu") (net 5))
 (segment (start 137.5625 106.7) (end 138.2 106.7) (width 0.2) (layer "F.Cu") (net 5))
 (segment (start 139.4375 95.5) (end 140.9375 97) (width 0.2) (layer "F.Cu") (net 5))
 (segment (start 137.5625 106.7) (end 137.5625 105.5) (width 0.2) (layer "F.Cu") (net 5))
 (segment (start 154.4125 113.5) (end 154.4125 110.475) (width 0.2) (layer "F.Cu") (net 5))
 (segment (start 139.4375 98.2625) (end 139.4375 95.5) (width 0.2) (layer "F.Cu") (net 5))
 (segment (start 149.4375 105.5) (end 150.35 105.5) (width 0.2) (layer "F.Cu") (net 5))
 (segment (start 151.6 86.8) (end 156.2625 86.8) (width 0.2) (layer "F.Cu") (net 5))
 (segment (start 150.35 105.5) (end 150.35 104.8) (width 0.2) (layer "F.Cu") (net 5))
 (segment (start 137.5625 105.5) (end 137.5625 104.3) (width 0.2) (layer "F.Cu") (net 5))
 (via (at 138.2 99.5) (size 0.6) (drill 0.3) (layers "F.Cu" "B.Cu") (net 5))
 (via (at 138.2 106.7) (size 0.6) (drill 0.3) (layers "F.Cu" "B.Cu") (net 5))
 (via (at 151.6 86.8) (size 0.6) (drill 0.3) (layers "F.Cu" "B.Cu") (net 5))
 (via (at 141.4 97) (size 0.6) (drill 0.3) (layers "F.Cu" "B.Cu") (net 5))
 (via (at 150.35 104.8) (size 0.6) (drill 0.3) (layers "F.Cu" "B.Cu") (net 5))
 (via (at 137.7 104.3) (size 0.6) (drill 0.3) (layers "F.Cu" "B.Cu") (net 5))
 (segment (start 150.35 104.8) (end 140.1 104.8) (width 0.2) (layer "B.Cu") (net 5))
 (segment (start 141.4 97) (end 151.6 86.8) (width 0.2) (layer "B.Cu") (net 5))
 (segment (start 137.7 104.3) (end 137.7 100) (width 0.2) (layer "B.Cu") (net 5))
 (segment (start 140.1 104.8) (end 138.2 106.7) (width 0.2) (layer "B.Cu") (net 5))
 (segment (start 137.7 100) (end 138.2 99.5) (width 0.2) (layer "B.Cu") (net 5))
 (segment (start 156.65 105.5) (end 156.65 104.8) (width 0.2) (layer "F.Cu") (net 10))
 (segment (start 164.4125 113.5) (end 157.5625 106.65) (width 0.2) (layer "F.Cu") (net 10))
 (segment (start 147.5625 95.5) (end 148.7625 96.7) (width 0.2) (layer "F.Cu") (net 10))
 (segment (start 159.4375 95.5) (end 159.4375 97.1375) (width 0.2) (layer "F.Cu") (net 10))
 (segment (start 159.4375 97.1375) (end 159.5 97.2) (width 0.2) (layer "F.Cu") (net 10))
 (segment (start 148.7625 96.7) (end 159.4375 96.7) (width 0.2) (layer "F.Cu") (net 10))
 (segment (start 157.5625 105.5) (end 156.65 105.5) (width 0.2) (layer "F.Cu") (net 10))
 (segment (start 157.5625 106.65) (end 157.5625 105.5) (width 0.2) (layer "F.Cu") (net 10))
 (via (at 156.65 104.8) (size 0.6) (drill 0.3) (layers "F.Cu" "B.Cu") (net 10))
 (via (at 159.5 97.2) (size 0.6) (drill 0.3) (layers "F.Cu" "B.Cu") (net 10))
 (segment (start 156.65 100.05) (end 156.65 104.8) (width 0.2) (layer "B.Cu") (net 10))
 (segment (start 159.5 97.2) (end 156.65 100.05) (width 0.2) (layer "B.Cu") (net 10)))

